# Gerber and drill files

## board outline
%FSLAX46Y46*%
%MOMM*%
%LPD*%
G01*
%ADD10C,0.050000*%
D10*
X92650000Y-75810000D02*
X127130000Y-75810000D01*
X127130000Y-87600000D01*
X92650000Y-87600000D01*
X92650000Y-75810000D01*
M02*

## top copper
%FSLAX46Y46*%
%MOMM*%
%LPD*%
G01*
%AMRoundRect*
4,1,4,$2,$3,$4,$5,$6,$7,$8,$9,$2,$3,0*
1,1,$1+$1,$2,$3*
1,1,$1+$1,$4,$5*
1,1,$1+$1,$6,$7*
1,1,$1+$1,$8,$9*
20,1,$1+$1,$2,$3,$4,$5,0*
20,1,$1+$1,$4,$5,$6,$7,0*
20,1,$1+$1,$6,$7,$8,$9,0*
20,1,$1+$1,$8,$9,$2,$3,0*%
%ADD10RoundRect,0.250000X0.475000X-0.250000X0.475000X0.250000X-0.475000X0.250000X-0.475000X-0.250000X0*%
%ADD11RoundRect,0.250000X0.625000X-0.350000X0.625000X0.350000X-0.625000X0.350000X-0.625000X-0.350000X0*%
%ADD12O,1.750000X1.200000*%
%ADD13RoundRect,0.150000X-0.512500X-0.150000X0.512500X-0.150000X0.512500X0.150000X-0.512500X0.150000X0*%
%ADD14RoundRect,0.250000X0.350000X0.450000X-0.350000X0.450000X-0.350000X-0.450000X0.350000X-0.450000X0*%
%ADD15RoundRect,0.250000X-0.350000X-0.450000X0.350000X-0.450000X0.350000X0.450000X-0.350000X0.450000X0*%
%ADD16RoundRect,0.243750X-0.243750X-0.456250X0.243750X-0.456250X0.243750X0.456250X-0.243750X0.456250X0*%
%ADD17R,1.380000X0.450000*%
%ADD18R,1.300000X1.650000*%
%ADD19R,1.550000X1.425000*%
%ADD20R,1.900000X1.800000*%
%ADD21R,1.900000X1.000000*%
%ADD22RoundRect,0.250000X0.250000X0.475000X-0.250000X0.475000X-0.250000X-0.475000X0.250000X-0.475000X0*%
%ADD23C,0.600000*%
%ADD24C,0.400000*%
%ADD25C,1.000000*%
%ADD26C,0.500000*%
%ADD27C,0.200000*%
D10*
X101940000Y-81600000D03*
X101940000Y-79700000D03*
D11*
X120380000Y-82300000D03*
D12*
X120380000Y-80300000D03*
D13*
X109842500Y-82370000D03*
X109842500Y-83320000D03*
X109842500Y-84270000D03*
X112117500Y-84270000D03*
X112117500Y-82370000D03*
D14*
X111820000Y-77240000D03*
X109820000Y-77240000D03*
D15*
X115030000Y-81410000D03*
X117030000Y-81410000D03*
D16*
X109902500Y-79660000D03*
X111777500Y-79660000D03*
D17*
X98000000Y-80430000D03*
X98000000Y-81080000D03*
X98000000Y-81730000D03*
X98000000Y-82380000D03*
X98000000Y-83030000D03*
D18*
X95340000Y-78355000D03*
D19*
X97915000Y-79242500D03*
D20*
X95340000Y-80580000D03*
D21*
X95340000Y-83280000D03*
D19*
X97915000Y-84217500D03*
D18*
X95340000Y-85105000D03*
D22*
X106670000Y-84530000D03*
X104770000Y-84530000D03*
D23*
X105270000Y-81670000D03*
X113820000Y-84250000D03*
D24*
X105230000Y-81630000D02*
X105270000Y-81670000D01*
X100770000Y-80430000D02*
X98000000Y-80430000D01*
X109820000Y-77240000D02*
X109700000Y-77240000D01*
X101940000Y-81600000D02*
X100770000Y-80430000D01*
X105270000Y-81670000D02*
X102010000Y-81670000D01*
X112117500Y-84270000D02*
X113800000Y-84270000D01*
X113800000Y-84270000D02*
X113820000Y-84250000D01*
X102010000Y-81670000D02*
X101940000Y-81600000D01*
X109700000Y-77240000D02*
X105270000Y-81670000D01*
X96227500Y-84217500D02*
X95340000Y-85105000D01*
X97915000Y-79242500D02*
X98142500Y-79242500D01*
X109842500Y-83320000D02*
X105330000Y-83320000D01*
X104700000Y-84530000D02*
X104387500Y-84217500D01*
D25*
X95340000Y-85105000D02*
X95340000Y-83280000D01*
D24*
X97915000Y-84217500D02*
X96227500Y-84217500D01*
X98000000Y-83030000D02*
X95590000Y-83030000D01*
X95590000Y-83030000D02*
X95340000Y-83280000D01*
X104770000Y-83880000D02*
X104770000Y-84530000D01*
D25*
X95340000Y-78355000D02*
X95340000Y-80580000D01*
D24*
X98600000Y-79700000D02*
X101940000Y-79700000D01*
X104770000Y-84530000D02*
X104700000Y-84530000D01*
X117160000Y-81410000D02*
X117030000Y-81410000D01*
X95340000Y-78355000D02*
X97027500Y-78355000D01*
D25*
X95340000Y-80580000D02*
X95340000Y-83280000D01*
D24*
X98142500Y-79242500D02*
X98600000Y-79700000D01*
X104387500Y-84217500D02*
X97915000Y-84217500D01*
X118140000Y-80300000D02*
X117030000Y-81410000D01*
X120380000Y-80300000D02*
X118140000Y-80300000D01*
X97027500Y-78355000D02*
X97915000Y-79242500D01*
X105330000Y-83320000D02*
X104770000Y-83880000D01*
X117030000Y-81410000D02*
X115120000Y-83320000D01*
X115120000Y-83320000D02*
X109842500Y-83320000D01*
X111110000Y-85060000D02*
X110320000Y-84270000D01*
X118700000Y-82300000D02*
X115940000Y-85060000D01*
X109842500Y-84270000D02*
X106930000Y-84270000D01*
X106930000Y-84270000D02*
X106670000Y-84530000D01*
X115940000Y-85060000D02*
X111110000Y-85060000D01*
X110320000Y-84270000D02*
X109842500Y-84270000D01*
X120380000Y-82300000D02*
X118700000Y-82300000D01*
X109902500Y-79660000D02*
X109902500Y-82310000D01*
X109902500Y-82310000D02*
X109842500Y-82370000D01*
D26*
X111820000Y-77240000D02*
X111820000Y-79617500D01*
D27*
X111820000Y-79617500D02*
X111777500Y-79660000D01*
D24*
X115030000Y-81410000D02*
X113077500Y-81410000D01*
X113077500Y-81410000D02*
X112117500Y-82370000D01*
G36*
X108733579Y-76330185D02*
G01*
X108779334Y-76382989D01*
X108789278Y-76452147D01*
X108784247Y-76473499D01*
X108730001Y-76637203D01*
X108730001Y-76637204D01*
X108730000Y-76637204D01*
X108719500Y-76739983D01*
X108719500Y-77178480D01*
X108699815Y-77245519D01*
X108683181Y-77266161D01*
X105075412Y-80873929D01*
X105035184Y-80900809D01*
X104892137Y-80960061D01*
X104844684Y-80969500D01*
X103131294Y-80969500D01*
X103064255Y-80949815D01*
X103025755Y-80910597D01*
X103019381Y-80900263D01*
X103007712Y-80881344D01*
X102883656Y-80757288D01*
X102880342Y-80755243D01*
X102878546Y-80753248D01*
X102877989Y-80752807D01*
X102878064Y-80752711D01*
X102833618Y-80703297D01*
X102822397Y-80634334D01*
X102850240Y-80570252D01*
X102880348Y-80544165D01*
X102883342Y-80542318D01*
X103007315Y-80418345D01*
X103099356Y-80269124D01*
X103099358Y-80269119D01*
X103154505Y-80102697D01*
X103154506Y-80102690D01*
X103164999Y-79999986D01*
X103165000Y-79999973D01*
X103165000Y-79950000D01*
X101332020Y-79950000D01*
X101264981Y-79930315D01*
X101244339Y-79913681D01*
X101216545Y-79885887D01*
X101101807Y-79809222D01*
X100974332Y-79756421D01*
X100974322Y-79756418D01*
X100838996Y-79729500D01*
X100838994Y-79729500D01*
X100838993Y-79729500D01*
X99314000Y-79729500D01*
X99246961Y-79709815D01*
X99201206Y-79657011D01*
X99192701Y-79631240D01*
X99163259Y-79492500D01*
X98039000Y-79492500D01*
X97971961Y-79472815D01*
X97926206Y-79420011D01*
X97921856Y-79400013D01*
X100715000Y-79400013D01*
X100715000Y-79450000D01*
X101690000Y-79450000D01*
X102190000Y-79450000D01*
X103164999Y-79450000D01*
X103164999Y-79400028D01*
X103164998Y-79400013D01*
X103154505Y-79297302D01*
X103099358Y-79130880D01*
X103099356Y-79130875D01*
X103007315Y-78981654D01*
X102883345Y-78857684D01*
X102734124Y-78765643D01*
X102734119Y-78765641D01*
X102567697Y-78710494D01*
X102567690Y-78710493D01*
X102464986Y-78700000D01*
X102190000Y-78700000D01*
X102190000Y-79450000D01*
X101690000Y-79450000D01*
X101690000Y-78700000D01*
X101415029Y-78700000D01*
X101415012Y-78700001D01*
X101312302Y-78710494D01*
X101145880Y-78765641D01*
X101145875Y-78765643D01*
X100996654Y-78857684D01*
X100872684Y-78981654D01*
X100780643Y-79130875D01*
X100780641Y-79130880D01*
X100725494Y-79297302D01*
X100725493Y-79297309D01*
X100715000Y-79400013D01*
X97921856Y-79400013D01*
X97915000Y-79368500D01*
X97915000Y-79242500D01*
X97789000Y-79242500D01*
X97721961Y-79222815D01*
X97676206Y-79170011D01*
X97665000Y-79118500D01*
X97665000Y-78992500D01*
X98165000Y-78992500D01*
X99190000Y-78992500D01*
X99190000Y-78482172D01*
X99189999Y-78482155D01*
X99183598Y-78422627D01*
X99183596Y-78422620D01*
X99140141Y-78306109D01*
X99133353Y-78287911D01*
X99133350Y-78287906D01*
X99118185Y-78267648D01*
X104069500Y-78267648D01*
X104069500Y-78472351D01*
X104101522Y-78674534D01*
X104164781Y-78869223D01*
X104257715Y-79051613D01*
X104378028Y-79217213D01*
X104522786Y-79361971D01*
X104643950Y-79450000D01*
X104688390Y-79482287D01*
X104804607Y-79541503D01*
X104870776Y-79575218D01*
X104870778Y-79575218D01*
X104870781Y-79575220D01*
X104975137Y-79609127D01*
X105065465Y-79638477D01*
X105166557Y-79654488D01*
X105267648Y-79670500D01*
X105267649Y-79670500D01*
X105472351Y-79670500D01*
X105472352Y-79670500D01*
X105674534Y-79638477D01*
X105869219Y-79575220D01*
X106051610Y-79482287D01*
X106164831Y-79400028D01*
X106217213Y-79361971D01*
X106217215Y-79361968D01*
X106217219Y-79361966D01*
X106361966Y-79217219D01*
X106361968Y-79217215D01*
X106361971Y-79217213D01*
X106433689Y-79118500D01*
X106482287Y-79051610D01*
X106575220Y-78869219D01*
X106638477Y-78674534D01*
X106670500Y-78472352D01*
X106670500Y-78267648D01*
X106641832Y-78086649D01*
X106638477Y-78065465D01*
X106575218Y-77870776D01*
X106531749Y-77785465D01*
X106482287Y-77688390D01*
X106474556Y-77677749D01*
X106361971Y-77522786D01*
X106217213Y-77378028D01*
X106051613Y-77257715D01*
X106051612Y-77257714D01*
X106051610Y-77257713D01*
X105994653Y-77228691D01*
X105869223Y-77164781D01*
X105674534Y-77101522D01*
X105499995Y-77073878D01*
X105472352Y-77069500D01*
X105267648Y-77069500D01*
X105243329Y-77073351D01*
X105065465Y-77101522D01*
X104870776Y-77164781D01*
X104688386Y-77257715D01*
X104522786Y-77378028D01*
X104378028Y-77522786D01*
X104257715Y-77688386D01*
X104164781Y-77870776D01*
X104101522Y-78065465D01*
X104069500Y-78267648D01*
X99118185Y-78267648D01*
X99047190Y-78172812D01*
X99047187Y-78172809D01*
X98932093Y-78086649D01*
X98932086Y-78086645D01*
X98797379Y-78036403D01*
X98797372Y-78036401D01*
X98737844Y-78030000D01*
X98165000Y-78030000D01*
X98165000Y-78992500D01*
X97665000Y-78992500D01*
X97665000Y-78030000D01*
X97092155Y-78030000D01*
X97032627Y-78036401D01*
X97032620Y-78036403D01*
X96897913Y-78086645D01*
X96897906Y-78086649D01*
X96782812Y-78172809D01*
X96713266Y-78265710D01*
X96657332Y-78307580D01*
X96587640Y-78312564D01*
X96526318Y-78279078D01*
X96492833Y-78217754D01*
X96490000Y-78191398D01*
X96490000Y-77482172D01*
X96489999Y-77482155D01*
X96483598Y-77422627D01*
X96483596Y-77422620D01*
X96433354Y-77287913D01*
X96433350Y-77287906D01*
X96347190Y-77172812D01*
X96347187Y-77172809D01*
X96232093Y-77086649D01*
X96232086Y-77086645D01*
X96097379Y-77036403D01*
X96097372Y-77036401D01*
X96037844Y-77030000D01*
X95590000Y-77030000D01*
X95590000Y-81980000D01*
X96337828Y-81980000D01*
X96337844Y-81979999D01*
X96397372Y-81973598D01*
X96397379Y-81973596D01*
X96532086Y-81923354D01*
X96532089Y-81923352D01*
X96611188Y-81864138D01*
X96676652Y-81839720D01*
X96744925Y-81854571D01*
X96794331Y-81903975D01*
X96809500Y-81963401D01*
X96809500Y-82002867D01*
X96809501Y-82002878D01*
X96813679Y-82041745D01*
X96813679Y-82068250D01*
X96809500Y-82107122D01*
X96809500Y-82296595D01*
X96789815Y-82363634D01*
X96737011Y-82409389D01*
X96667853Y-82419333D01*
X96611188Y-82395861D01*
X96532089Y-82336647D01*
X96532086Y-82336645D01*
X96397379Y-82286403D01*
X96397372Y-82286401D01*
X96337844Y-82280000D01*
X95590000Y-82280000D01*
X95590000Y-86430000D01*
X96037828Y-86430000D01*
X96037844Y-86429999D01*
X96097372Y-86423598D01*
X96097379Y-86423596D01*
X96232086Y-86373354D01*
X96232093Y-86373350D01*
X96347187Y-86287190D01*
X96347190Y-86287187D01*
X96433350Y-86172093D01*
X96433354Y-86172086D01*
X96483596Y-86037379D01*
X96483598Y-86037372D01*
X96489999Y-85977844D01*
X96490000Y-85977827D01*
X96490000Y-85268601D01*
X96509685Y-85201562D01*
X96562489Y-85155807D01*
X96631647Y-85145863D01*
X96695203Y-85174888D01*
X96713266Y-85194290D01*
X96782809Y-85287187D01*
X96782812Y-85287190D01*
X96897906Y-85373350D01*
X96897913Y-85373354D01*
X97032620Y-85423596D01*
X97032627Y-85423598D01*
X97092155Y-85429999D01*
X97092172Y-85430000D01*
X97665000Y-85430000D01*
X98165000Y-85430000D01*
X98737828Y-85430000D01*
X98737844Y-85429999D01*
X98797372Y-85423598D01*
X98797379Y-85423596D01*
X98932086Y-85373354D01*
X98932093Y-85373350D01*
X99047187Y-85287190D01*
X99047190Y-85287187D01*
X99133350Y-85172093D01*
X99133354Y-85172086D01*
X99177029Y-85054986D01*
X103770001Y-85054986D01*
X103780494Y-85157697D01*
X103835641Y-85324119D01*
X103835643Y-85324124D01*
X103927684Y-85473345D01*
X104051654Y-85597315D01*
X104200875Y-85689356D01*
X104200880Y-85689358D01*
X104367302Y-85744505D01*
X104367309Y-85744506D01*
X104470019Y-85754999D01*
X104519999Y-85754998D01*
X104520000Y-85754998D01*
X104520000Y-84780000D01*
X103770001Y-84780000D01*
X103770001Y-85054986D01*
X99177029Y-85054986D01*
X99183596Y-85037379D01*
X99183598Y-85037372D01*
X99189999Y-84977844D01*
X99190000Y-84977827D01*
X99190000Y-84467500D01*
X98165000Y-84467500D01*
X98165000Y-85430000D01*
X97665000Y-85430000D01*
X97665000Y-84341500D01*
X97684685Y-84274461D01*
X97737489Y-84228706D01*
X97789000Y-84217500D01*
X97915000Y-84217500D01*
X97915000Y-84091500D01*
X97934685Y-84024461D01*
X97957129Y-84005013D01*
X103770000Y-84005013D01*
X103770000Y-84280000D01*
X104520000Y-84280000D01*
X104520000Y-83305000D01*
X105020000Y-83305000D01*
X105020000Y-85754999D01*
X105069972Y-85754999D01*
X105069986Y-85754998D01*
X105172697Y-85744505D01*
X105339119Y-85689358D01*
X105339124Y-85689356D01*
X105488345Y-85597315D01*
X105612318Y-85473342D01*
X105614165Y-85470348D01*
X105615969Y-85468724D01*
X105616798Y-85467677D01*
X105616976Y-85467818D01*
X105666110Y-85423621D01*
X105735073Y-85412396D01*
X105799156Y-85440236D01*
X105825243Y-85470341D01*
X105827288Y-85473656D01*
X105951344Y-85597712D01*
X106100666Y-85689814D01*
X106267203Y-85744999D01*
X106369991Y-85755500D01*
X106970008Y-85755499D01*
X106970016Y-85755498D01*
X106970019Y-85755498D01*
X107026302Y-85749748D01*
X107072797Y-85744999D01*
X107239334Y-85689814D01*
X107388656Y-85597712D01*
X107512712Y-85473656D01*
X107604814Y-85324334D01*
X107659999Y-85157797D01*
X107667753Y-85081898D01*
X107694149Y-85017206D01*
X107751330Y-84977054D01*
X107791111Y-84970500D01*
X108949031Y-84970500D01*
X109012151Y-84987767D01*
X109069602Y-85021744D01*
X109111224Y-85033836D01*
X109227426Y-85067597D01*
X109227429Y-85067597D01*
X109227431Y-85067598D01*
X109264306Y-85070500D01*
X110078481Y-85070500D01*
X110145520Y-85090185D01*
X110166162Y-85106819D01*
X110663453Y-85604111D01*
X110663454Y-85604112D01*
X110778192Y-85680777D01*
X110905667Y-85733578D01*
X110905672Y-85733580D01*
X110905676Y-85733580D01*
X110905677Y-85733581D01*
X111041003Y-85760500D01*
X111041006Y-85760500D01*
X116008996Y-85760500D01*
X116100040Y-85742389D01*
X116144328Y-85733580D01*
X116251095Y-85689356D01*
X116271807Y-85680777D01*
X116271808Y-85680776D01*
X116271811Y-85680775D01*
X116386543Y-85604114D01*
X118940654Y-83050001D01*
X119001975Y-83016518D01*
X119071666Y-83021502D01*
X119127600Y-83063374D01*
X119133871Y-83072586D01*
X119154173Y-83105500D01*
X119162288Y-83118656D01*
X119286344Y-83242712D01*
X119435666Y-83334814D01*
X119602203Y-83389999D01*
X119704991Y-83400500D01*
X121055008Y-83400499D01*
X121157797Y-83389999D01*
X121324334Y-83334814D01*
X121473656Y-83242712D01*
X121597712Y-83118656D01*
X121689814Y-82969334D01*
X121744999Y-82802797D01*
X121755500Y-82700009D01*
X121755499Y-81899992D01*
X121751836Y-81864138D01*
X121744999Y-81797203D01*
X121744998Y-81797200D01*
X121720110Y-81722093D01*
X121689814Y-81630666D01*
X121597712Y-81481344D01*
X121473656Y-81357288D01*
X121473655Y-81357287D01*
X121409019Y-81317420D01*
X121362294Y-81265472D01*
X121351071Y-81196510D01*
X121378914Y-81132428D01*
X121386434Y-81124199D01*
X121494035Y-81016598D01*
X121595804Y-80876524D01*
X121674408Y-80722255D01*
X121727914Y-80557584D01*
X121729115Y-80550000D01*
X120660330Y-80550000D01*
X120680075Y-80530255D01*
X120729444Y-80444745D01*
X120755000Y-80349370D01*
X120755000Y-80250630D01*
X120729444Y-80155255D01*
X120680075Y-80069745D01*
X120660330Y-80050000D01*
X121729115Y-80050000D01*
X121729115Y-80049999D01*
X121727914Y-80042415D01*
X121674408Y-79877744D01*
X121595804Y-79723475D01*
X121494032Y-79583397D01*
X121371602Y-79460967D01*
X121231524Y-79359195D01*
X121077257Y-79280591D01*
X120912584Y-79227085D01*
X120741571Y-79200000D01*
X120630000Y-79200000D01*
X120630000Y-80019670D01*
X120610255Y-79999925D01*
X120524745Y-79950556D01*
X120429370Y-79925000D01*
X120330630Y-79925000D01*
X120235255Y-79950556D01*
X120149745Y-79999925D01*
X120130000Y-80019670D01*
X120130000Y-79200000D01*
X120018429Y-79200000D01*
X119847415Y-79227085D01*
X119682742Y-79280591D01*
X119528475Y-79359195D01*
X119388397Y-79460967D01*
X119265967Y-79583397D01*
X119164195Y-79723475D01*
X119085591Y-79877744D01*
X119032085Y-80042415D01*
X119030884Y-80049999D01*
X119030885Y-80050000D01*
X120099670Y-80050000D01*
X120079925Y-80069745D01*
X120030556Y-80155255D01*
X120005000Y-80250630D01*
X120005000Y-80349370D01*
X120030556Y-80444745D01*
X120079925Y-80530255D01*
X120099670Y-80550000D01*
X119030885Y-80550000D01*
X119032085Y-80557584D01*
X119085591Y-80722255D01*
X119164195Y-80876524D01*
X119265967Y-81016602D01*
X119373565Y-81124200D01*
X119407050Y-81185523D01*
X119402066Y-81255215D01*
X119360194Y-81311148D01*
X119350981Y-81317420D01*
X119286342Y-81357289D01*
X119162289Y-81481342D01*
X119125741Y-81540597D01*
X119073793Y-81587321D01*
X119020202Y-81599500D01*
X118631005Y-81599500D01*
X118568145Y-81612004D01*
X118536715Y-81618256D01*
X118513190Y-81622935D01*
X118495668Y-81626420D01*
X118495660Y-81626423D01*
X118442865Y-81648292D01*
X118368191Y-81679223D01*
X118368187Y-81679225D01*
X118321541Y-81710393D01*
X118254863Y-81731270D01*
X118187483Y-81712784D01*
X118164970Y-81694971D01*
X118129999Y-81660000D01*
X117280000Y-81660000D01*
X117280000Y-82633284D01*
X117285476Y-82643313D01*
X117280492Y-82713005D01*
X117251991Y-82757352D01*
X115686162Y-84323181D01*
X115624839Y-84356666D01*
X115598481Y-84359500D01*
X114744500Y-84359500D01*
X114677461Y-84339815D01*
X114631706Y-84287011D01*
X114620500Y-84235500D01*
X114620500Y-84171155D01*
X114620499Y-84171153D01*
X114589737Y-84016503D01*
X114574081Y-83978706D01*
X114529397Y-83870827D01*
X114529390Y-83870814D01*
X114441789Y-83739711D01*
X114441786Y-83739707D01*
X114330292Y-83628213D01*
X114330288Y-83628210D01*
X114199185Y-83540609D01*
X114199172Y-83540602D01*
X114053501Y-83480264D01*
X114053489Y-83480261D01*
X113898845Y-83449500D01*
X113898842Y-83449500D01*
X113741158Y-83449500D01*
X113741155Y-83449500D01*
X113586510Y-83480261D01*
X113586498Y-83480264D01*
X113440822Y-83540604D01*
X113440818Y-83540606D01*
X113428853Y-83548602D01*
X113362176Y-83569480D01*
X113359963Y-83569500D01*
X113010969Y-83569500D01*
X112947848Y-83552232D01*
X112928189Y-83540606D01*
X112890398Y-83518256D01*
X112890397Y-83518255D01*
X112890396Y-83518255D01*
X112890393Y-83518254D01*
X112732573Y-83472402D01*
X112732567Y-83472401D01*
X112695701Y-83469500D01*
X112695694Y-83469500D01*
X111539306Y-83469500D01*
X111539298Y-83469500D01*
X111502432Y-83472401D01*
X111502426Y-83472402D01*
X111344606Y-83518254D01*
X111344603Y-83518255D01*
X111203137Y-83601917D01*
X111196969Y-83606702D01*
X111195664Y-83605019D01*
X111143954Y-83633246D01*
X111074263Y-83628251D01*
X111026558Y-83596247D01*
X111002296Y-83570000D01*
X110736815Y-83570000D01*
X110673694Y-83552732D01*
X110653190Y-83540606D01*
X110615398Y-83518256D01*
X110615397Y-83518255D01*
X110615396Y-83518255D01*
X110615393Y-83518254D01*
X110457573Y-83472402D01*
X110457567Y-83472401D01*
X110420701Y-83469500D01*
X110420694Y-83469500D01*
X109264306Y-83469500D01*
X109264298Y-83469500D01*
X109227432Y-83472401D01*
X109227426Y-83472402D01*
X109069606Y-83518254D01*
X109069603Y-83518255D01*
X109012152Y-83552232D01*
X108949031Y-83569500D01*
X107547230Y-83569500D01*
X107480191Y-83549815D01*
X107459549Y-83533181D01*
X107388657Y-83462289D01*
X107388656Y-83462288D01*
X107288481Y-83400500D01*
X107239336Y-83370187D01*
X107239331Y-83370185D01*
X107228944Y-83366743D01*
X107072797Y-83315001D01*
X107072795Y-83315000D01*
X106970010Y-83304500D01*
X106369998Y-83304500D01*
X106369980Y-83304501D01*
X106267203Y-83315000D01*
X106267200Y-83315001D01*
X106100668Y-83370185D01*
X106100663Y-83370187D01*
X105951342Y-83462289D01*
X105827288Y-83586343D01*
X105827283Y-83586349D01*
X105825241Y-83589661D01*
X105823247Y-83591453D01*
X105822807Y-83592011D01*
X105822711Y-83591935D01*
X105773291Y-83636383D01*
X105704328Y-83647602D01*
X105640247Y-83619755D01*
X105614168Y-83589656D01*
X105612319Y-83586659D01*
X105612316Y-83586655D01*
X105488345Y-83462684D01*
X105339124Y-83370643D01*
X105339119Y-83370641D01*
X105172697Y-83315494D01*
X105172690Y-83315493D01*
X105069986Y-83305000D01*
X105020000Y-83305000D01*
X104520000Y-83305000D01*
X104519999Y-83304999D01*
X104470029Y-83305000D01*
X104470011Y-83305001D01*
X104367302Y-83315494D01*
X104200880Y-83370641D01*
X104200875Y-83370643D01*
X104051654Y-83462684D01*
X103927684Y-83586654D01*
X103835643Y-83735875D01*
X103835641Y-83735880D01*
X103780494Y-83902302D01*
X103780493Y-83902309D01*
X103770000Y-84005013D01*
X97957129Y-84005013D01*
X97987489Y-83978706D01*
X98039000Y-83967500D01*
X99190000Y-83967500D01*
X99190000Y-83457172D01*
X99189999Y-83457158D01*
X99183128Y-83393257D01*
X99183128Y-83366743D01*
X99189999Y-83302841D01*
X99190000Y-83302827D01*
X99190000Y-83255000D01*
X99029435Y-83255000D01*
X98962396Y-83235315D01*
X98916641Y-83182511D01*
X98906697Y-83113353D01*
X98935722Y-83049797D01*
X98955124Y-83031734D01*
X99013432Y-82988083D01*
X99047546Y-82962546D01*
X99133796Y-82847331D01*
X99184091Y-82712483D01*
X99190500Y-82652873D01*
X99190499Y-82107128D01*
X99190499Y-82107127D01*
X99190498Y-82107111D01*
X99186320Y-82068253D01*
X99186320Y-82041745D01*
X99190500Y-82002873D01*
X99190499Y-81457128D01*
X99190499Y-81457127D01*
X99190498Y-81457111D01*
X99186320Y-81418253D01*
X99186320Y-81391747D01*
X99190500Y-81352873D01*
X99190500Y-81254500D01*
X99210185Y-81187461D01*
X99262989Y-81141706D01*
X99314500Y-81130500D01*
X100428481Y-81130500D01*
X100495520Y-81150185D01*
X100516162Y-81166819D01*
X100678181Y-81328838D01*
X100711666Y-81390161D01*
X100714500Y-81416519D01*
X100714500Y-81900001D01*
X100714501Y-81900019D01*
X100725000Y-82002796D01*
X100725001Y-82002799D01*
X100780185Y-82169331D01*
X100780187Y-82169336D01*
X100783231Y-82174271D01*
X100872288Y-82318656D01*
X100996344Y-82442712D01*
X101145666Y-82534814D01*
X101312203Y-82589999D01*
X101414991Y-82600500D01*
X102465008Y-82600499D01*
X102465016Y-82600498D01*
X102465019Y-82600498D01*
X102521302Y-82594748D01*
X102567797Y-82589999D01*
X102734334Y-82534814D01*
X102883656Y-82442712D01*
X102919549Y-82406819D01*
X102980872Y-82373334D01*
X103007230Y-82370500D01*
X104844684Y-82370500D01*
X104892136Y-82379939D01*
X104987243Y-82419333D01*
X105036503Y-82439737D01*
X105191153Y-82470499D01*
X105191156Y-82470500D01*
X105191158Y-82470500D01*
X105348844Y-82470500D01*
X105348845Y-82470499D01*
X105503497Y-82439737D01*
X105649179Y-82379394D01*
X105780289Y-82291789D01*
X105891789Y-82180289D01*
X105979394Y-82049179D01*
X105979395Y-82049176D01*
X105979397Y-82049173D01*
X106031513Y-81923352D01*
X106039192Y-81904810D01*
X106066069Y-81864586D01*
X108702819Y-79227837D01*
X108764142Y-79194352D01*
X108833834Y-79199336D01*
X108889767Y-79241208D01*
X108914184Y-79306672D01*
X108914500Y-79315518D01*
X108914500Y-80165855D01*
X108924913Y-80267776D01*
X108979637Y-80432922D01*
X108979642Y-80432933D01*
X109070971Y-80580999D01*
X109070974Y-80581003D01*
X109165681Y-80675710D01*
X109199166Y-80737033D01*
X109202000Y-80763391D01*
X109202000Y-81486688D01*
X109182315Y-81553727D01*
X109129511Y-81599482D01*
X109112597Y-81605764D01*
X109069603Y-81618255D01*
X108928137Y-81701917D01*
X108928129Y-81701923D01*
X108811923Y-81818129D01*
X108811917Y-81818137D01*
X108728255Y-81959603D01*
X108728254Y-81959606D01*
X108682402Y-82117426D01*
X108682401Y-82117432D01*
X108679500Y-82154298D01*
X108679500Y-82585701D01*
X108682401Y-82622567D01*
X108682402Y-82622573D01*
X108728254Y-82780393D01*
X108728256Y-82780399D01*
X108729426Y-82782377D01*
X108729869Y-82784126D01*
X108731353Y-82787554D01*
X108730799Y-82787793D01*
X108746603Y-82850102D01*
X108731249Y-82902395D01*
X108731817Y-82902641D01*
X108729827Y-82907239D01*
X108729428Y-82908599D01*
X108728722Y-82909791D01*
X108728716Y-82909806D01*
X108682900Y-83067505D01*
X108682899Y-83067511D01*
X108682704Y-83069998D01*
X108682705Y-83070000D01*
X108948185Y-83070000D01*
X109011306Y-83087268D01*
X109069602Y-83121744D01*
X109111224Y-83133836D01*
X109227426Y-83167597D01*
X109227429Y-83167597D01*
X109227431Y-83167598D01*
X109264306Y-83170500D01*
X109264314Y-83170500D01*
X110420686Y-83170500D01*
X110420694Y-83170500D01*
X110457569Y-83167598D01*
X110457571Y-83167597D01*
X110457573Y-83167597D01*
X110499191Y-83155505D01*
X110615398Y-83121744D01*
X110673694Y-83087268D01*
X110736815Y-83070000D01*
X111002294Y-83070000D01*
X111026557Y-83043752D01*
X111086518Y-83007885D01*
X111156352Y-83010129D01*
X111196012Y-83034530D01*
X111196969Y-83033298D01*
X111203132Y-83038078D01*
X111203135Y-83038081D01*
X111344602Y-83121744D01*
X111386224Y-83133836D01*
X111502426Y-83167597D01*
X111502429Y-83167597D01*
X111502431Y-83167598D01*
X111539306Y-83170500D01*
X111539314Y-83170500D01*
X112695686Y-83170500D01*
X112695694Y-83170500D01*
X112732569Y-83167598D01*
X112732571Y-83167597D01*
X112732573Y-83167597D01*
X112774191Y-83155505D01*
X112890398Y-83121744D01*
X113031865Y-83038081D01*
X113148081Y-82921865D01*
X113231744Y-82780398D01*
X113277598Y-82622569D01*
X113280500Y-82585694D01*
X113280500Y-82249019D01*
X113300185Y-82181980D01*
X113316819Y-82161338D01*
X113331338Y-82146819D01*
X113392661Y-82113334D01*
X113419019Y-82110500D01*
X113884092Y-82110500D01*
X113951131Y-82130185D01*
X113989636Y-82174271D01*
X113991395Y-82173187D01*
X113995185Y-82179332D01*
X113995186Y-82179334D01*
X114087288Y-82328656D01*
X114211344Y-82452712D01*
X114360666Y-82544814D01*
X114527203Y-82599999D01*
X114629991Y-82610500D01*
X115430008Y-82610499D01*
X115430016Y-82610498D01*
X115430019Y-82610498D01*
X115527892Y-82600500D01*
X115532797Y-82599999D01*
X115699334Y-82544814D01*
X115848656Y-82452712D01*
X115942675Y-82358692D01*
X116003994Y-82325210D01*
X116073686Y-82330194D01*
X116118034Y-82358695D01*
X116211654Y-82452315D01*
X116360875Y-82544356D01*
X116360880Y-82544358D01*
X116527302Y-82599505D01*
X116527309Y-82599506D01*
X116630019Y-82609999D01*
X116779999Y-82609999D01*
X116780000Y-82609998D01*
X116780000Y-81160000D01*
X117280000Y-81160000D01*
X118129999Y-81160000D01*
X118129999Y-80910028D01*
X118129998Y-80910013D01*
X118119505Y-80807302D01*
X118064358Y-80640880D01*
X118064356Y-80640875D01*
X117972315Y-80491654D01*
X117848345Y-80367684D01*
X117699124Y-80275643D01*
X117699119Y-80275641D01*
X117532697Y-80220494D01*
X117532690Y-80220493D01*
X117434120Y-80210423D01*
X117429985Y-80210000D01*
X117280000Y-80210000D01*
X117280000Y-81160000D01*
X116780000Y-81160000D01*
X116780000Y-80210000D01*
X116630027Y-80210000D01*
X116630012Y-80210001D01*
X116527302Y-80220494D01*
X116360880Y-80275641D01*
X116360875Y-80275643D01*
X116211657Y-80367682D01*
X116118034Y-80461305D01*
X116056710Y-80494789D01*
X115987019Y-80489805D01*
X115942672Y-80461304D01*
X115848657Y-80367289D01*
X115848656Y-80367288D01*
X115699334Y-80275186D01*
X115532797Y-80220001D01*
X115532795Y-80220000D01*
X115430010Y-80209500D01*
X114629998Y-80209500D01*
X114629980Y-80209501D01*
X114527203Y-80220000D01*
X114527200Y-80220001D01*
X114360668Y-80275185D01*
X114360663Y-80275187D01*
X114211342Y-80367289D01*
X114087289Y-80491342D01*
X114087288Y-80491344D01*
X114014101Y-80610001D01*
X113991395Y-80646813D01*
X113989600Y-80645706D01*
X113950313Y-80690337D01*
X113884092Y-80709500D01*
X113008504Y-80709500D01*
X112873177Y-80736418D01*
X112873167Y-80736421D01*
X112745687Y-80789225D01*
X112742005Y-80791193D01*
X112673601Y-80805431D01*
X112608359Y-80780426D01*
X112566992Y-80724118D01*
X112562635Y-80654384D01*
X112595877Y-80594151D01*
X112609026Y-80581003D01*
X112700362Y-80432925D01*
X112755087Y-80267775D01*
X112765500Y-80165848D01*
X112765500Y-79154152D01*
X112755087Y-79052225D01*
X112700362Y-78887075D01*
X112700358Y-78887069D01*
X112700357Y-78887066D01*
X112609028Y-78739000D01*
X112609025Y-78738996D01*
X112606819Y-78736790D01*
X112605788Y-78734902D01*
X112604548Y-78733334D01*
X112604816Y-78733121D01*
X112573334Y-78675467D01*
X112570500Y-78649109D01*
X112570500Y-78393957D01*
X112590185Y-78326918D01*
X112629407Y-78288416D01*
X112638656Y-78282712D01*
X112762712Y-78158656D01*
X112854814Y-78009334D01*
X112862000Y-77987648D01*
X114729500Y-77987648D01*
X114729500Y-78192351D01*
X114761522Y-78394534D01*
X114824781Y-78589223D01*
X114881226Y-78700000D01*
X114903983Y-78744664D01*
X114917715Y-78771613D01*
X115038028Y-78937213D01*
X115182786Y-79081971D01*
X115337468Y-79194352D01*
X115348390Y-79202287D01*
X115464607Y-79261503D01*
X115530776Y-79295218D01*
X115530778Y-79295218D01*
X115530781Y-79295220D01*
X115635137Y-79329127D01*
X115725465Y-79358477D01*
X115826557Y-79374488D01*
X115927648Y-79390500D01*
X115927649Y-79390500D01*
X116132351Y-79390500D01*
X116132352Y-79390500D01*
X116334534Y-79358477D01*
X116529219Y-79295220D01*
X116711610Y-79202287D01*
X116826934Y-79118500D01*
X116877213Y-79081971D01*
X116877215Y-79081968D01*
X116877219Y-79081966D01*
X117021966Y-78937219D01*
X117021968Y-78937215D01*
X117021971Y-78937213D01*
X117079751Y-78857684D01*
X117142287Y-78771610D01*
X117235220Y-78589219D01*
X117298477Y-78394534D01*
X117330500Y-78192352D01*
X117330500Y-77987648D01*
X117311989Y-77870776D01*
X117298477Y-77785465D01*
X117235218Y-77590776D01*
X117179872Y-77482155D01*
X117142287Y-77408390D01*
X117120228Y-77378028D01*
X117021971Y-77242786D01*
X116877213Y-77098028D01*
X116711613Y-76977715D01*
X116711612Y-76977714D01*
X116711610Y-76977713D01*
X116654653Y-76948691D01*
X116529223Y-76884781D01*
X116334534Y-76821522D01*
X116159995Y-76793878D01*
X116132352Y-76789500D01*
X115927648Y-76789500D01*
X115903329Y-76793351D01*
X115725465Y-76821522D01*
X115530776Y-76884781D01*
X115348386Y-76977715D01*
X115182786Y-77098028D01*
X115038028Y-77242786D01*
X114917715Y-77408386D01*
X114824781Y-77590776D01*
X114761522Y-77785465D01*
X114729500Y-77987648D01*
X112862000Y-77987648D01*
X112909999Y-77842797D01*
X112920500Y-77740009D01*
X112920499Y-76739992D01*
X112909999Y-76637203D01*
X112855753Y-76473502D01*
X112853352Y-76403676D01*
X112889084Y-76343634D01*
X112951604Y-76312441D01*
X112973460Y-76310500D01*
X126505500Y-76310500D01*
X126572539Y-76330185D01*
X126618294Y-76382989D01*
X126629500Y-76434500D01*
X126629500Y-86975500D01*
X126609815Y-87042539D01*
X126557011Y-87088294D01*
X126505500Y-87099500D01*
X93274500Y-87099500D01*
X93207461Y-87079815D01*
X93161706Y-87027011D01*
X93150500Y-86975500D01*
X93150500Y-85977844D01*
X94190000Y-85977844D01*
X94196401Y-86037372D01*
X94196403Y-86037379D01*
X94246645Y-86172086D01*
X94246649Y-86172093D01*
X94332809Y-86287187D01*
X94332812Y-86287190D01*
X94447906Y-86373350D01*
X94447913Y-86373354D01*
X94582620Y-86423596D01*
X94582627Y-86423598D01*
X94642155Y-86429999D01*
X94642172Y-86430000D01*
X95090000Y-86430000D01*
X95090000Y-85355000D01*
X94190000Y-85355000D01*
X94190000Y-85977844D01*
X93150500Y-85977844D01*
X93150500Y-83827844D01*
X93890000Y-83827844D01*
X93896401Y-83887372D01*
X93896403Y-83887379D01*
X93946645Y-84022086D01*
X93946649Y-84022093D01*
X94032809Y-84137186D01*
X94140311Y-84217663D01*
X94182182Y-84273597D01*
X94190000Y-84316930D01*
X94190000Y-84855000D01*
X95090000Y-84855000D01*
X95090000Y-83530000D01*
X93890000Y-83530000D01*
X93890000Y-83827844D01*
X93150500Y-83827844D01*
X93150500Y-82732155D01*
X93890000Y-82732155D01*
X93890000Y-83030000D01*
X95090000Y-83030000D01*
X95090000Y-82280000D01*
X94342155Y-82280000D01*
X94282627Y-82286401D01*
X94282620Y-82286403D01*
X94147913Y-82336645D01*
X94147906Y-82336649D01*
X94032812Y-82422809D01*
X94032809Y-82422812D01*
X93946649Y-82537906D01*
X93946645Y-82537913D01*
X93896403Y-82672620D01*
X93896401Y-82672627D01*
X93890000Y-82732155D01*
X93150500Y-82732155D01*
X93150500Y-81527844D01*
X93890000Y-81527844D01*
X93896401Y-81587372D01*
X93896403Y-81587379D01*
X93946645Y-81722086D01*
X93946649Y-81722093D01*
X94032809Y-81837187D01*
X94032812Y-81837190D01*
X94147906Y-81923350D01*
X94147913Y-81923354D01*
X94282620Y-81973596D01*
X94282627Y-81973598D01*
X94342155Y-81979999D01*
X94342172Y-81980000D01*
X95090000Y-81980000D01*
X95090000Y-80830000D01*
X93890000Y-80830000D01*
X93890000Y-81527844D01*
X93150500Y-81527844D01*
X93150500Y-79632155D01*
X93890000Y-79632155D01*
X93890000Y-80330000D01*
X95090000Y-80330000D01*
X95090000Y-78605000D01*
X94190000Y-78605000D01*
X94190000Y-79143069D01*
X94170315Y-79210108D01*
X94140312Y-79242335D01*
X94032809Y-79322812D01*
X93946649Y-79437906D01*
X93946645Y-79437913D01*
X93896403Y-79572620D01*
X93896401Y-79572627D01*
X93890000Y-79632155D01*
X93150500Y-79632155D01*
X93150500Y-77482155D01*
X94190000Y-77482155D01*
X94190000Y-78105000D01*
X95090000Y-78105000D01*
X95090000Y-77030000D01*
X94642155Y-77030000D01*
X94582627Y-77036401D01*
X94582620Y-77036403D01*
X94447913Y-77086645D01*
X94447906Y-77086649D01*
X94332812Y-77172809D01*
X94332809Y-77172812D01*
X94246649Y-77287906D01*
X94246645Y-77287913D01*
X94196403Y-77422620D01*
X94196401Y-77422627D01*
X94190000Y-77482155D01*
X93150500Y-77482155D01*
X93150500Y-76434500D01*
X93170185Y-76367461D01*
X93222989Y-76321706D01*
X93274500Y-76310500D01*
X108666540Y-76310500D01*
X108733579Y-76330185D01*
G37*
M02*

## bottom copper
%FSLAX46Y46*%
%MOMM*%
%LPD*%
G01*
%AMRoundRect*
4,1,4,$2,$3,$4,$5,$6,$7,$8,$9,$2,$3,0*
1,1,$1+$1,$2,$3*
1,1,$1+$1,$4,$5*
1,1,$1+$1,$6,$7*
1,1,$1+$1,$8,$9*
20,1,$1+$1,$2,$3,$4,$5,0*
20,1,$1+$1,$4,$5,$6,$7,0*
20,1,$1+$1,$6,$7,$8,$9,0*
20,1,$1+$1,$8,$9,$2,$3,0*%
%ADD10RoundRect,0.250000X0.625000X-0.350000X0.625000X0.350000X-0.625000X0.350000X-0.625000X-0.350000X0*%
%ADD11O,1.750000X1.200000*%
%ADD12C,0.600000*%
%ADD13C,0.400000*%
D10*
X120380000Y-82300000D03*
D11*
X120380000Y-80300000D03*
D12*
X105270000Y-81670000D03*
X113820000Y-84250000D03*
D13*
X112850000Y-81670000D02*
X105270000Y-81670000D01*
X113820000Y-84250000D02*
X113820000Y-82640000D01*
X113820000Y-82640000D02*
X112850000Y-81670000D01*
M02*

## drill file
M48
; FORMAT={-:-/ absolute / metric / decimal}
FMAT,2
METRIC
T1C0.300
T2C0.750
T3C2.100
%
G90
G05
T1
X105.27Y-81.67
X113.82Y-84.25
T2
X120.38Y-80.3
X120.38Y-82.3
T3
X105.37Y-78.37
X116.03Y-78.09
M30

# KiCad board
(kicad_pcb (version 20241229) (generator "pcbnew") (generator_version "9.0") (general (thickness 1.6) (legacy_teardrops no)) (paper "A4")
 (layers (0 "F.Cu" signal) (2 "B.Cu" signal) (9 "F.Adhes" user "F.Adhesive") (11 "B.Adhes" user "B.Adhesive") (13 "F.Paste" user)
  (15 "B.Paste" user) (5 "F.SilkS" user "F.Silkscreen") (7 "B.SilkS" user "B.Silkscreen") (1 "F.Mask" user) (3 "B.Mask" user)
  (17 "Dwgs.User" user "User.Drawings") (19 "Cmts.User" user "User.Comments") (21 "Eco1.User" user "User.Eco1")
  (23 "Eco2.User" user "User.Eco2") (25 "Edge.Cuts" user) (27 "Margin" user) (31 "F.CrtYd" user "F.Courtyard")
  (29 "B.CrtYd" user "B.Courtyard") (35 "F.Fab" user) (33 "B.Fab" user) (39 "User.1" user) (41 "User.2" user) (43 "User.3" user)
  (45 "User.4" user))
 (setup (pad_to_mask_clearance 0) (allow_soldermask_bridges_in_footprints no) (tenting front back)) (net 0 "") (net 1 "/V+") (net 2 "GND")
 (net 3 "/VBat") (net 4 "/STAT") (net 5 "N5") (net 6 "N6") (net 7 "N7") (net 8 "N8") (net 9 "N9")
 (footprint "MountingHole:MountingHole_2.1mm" (layer "F.Cu") (at 105.37 78.37)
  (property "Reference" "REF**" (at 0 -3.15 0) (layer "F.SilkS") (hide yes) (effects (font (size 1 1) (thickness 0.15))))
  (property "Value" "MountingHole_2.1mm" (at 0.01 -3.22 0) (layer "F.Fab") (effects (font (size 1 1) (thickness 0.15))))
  (pad "" np_thru_hole circle (at 0 0) (size 2.1 2.1) (drill 2.1) (layers "*.Cu" "*.Mask")))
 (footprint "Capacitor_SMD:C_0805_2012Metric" (layer "F.Cu") (at 101.94 80.65 90)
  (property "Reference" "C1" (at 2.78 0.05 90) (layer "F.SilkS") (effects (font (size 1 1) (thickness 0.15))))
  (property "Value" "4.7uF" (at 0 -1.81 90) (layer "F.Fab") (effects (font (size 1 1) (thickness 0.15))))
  (pad "1" smd roundrect (at -0.95 0 90) (size 1 1.45) (layers "F.Cu" "F.Mask" "F.Paste") (roundrect_rratio 0.25) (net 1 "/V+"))
  (pad "2" smd roundrect (at 0.95 0 90) (size 1 1.45) (layers "F.Cu" "F.Mask" "F.Paste") (roundrect_rratio 0.25) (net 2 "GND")))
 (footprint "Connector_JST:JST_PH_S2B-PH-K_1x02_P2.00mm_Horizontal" (layer "F.Cu") (at 120.38 82.3 90)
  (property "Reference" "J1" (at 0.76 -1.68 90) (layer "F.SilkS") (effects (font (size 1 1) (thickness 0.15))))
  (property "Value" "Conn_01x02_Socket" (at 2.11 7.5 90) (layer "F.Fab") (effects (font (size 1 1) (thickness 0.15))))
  (pad "1" thru_hole roundrect (at 0 0 90) (size 1.2 1.75) (drill 0.75) (layers "*.Cu" "*.Mask") (remove_unused_layers no)
   (roundrect_rratio 0.208333) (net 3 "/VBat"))
  (pad "2" thru_hole oval (at 2 0 90) (size 1.2 1.75) (drill 0.75) (layers "*.Cu" "*.Mask") (remove_unused_layers no) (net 2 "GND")))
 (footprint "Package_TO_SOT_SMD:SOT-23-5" (layer "F.Cu") (at 110.98 83.32)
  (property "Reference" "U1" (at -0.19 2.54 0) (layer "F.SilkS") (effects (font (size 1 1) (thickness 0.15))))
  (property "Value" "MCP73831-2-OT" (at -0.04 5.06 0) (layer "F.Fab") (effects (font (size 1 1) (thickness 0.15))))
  (pad "1" smd roundrect (at -1.1375 -0.95) (size 1.325 0.6) (layers "F.Cu" "F.Mask" "F.Paste") (roundrect_rratio 0.25) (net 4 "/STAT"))
  (pad "2" smd roundrect (at -1.1375 0) (size 1.325 0.6) (layers "F.Cu" "F.Mask" "F.Paste") (roundrect_rratio 0.25) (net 2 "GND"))
  (pad "3" smd roundrect (at -1.1375 0.95) (size 1.325 0.6) (layers "F.Cu" "F.Mask" "F.Paste") (roundrect_rratio 0.25) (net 3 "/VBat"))
  (pad "4" smd roundrect (at 1.1375 0.95) (size 1.325 0.6) (layers "F.Cu" "F.Mask" "F.Paste") (roundrect_rratio 0.25) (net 1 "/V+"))
  (pad "5" smd roundrect (at 1.1375 -0.95) (size 1.325 0.6) (layers "F.Cu" "F.Mask" "F.Paste") (roundrect_rratio 0.25) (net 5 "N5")))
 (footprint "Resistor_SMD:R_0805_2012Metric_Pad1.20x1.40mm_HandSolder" (layer "F.Cu") (at 110.82 77.24 180)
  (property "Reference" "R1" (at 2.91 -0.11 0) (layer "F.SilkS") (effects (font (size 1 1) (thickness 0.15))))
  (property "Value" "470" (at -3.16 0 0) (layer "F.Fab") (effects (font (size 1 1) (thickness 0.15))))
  (pad "1" smd roundrect (at -1 0 180) (size 1.2 1.4) (layers "F.Cu" "F.Mask" "F.Paste") (roundrect_rratio 0.208333) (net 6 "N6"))
  (pad "2" smd roundrect (at 1 0 180) (size 1.2 1.4) (layers "F.Cu" "F.Mask" "F.Paste") (roundrect_rratio 0.208333) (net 1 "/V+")))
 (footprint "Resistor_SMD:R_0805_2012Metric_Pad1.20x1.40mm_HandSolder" (layer "F.Cu") (at 116.03 81.41)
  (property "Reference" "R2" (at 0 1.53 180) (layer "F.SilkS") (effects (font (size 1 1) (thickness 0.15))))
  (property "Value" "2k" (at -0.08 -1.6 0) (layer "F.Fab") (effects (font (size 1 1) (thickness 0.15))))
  (pad "1" smd roundrect (at -1 0) (size 1.2 1.4) (layers "F.Cu" "F.Mask" "F.Paste") (roundrect_rratio 0.208333) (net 5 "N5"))
  (pad "2" smd roundrect (at 1 0) (size 1.2 1.4) (layers "F.Cu" "F.Mask" "F.Paste") (roundrect_rratio 0.208333) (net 2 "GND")))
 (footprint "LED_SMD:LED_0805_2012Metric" (layer "F.Cu") (at 110.84 79.66)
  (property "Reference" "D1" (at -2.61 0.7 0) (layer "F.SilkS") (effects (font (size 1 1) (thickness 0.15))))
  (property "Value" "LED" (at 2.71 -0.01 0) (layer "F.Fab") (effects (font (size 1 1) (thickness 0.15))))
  (pad "1" smd roundrect (at -0.9375 0) (size 0.975 1.4) (layers "F.Cu" "F.Mask" "F.Paste") (roundrect_rratio 0.25) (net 4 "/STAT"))
  (pad "2" smd roundrect (at 0.9375 0) (size 0.975 1.4) (layers "F.Cu" "F.Mask" "F.Paste") (roundrect_rratio 0.25) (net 6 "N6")))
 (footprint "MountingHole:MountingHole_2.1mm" (layer "F.Cu") (at 116.03 78.09)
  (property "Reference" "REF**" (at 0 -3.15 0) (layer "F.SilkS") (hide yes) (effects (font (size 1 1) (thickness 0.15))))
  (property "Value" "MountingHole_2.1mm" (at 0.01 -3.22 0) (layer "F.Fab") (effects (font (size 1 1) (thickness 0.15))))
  (pad "" np_thru_hole circle (at 0 0) (size 2.1 2.1) (drill 2.1) (layers "*.Cu" "*.Mask")))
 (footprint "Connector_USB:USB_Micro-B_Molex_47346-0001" (layer "F.Cu") (at 96.54 81.73 -90)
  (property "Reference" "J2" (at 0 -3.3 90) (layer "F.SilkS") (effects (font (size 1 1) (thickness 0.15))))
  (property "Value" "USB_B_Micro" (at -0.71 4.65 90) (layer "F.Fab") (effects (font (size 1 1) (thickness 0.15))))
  (pad "1" smd rect (at -1.3 -1.46 270) (size 0.45 1.38) (layers "F.Cu" "F.Mask" "F.Paste") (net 1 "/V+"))
  (pad "2" smd rect (at -0.65 -1.46 270) (size 0.45 1.38) (layers "F.Cu" "F.Mask" "F.Paste") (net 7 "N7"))
  (pad "3" smd rect (at 0 -1.46 270) (size 0.45 1.38) (layers "F.Cu" "F.Mask" "F.Paste") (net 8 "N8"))
  (pad "4" smd rect (at 0.65 -1.46 270) (size 0.45 1.38) (layers "F.Cu" "F.Mask" "F.Paste") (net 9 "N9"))
  (pad "5" smd rect (at 1.3 -1.46 270) (size 0.45 1.38) (layers "F.Cu" "F.Mask" "F.Paste") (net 2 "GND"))
  (pad "6" smd rect (at -3.375 1.2 270) (size 1.65 1.3) (layers "F.Cu" "F.Mask" "F.Paste") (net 2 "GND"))
  (pad "6" smd rect (at -2.4875 -1.375 270) (size 1.425 1.55) (layers "F.Cu" "F.Mask" "F.Paste") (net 2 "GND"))
  (pad "6" smd rect (at -1.15 1.2 270) (size 1.8 1.9) (layers "F.Cu" "F.Mask" "F.Paste") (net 2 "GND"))
  (pad "6" smd rect (at 1.55 1.2 270) (size 1 1.9) (layers "F.Cu" "F.Mask" "F.Paste") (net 2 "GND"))
  (pad "6" smd rect (at 2.4875 -1.375 270) (size 1.425 1.55) (layers "F.Cu" "F.Mask" "F.Paste") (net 2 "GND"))
  (pad "6" smd rect (at 3.375 1.2 270) (size 1.65 1.3) (layers "F.Cu" "F.Mask" "F.Paste") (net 2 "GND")))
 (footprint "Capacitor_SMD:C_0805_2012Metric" (layer "F.Cu") (at 105.72 84.53 180)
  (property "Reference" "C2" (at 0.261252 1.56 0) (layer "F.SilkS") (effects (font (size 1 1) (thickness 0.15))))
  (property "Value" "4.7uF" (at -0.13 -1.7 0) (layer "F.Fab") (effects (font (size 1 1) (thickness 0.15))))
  (pad "1" smd roundrect (at -0.95 0 180) (size 1 1.45) (layers "F.Cu" "F.Mask" "F.Paste") (roundrect_rratio 0.25) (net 3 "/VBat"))
  (pad "2" smd roundrect (at 0.95 0 180) (size 1 1.45) (layers "F.Cu" "F.Mask" "F.Paste") (roundrect_rratio 0.25) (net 2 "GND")))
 (gr_rect (start 92.65 75.81) (end 127.13 87.6) (stroke (width 0.05) (type default)) (fill no) (layer "Edge.Cuts"))
 (segment (start 105.23 81.63) (end 105.27 81.67) (width 0.4) (layer "F.Cu") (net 1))
 (segment (start 100.77 80.43) (end 98 80.43) (width 0.4) (layer "F.Cu") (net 1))
 (segment (start 109.82 77.24) (end 109.7 77.24) (width 0.4) (layer "F.Cu") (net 1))
 (segment (start 101.94 81.6) (end 100.77 80.43) (width 0.4) (layer "F.Cu") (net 1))
 (segment (start 105.27 81.67) (end 102.01 81.67) (width 0.4) (layer "F.Cu") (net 1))
 (segment (start 112.1175 84.27) (end 113.8 84.27) (width 0.4) (layer "F.Cu") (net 1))
 (segment (start 113.8 84.27) (end 113.82 84.25) (width 0.4) (layer "F.Cu") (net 1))
 (segment (start 102.01 81.67) (end 101.94 81.6) (width 0.4) (layer "F.Cu") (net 1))
 (segment (start 109.7 77.24) (end 105.27 81.67) (width 0.4) (layer "F.Cu") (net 1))
 (via (at 105.27 81.67) (size 0.6) (drill 0.3) (layers "F.Cu" "B.Cu") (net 1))
 (via (at 113.82 84.25) (size 0.6) (drill 0.3) (layers "F.Cu" "B.Cu") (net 1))
 (segment (start 112.85 81.67) (end 105.27 81.67) (width 0.4) (layer "B.Cu") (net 1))
 (segment (start 113.82 84.25) (end 113.82 82.64) (width 0.4) (layer "B.Cu") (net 1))
 (segment (start 113.82 82.64) (end 112.85 81.67) (width 0.4) (layer "B.Cu") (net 1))
 (segment (start 96.2275 84.2175) (end 95.34 85.105) (width 0.4) (layer "F.Cu") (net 2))
 (segment (start 97.915 79.2425) (end 98.1425 79.2425) (width 0.4) (layer "F.Cu") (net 2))
 (segment (start 109.8425 83.32) (end 105.33 83.32) (width 0.4) (layer "F.Cu") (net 2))
 (segment (start 104.7 84.53) (end 104.3875 84.2175) (width 0.4) (layer "F.Cu") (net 2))
 (segment (start 95.34 85.105) (end 95.34 83.28) (width 1) (layer "F.Cu") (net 2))
 (segment (start 97.915 84.2175) (end 96.2275 84.2175) (width 0.4) (layer "F.Cu") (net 2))
 (segment (start 98 83.03) (end 95.59 83.03) (width 0.4) (layer "F.Cu") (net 2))
 (segment (start 95.59 83.03) (end 95.34 83.28) (width 0.4) (layer "F.Cu") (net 2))
 (segment (start 104.77 83.88) (end 104.77 84.53) (width 0.4) (layer "F.Cu") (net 2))
 (segment (start 95.34 78.355) (end 95.34 80.58) (width 1) (layer "F.Cu") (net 2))
 (segment (start 98.6 79.7) (end 101.94 79.7) (width 0.4) (layer "F.Cu") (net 2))
 (segment (start 104.77 84.53) (end 104.7 84.53) (width 0.4) (layer "F.Cu") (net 2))
 (segment (start 117.16 81.41) (end 117.03 81.41) (width 0.4) (layer "F.Cu") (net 2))
 (segment (start 95.34 78.355) (end 97.0275 78.355) (width 0.4) (layer "F.Cu") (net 2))
 (segment (start 95.34 80.58) (end 95.34 83.28) (width 1) (layer "F.Cu") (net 2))
 (segment (start 98.1425 79.2425) (end 98.6 79.7) (width 0.4) (layer "F.Cu") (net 2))
 (segment (start 104.3875 84.2175) (end 97.915 84.2175) (width 0.4) (layer "F.Cu") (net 2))
 (segment (start 118.14 80.3) (end 117.03 81.41) (width 0.4) (layer "F.Cu") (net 2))
 (segment (start 120.38 80.3) (end 118.14 80.3) (width 0.4) (layer "F.Cu") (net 2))
 (segment (start 97.0275 78.355) (end 97.915 79.2425) (width 0.4) (layer "F.Cu") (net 2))
 (segment (start 105.33 83.32) (end 104.77 83.88) (width 0.4) (layer "F.Cu") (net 2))
 (segment (start 117.03 81.41) (end 115.12 83.32) (width 0.4) (layer "F.Cu") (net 2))
 (segment (start 115.12 83.32) (end 109.8425 83.32) (width 0.4) (layer "F.Cu") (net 2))
 (segment (start 111.11 85.06) (end 110.32 84.27) (width 0.4) (layer "F.Cu") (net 3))
 (segment (start 118.7 82.3) (end 115.94 85.06) (width 0.4) (layer "F.Cu") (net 3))
 (segment (start 109.8425 84.27) (end 106.93 84.27) (width 0.4) (layer "F.Cu") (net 3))
 (segment (start 106.93 84.27) (end 106.67 84.53) (width 0.4) (layer "F.Cu") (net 3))
 (segment (start 115.94 85.06) (end 111.11 85.06) (width 0.4) (layer "F.Cu") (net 3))
 (segment (start 110.32 84.27) (end 109.8425 84.27) (width 0.4) (layer "F.Cu") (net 3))
 (segment (start 120.38 82.3) (end 118.7 82.3) (width 0.4) (layer "F.Cu") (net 3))
 (segment (start 109.9025 79.66) (end 109.9025 82.31) (width 0.4) (layer "F.Cu") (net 4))
 (segment (start 109.9025 82.31) (end 109.8425 82.37) (width 0.4) (layer "F.Cu") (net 4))
 (segment (start 111.82 77.24) (end 111.82 79.6175) (width 0.5) (layer "F.Cu") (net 6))
 (segment (start 111.82 79.6175) (end 111.7775 79.66) (width 0.2) (layer "F.Cu") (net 6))
 (segment (start 115.03 81.41) (end 113.0775 81.41) (width 0.4) (layer "F.Cu") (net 5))
 (segment (start 113.0775 81.41) (end 112.1175 82.37) (width 0.4) (layer "F.Cu") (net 5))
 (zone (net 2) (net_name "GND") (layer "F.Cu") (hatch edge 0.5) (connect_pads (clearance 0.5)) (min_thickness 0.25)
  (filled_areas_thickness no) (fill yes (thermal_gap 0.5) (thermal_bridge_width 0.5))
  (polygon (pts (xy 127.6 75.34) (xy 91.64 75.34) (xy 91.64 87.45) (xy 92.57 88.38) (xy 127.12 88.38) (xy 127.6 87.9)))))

